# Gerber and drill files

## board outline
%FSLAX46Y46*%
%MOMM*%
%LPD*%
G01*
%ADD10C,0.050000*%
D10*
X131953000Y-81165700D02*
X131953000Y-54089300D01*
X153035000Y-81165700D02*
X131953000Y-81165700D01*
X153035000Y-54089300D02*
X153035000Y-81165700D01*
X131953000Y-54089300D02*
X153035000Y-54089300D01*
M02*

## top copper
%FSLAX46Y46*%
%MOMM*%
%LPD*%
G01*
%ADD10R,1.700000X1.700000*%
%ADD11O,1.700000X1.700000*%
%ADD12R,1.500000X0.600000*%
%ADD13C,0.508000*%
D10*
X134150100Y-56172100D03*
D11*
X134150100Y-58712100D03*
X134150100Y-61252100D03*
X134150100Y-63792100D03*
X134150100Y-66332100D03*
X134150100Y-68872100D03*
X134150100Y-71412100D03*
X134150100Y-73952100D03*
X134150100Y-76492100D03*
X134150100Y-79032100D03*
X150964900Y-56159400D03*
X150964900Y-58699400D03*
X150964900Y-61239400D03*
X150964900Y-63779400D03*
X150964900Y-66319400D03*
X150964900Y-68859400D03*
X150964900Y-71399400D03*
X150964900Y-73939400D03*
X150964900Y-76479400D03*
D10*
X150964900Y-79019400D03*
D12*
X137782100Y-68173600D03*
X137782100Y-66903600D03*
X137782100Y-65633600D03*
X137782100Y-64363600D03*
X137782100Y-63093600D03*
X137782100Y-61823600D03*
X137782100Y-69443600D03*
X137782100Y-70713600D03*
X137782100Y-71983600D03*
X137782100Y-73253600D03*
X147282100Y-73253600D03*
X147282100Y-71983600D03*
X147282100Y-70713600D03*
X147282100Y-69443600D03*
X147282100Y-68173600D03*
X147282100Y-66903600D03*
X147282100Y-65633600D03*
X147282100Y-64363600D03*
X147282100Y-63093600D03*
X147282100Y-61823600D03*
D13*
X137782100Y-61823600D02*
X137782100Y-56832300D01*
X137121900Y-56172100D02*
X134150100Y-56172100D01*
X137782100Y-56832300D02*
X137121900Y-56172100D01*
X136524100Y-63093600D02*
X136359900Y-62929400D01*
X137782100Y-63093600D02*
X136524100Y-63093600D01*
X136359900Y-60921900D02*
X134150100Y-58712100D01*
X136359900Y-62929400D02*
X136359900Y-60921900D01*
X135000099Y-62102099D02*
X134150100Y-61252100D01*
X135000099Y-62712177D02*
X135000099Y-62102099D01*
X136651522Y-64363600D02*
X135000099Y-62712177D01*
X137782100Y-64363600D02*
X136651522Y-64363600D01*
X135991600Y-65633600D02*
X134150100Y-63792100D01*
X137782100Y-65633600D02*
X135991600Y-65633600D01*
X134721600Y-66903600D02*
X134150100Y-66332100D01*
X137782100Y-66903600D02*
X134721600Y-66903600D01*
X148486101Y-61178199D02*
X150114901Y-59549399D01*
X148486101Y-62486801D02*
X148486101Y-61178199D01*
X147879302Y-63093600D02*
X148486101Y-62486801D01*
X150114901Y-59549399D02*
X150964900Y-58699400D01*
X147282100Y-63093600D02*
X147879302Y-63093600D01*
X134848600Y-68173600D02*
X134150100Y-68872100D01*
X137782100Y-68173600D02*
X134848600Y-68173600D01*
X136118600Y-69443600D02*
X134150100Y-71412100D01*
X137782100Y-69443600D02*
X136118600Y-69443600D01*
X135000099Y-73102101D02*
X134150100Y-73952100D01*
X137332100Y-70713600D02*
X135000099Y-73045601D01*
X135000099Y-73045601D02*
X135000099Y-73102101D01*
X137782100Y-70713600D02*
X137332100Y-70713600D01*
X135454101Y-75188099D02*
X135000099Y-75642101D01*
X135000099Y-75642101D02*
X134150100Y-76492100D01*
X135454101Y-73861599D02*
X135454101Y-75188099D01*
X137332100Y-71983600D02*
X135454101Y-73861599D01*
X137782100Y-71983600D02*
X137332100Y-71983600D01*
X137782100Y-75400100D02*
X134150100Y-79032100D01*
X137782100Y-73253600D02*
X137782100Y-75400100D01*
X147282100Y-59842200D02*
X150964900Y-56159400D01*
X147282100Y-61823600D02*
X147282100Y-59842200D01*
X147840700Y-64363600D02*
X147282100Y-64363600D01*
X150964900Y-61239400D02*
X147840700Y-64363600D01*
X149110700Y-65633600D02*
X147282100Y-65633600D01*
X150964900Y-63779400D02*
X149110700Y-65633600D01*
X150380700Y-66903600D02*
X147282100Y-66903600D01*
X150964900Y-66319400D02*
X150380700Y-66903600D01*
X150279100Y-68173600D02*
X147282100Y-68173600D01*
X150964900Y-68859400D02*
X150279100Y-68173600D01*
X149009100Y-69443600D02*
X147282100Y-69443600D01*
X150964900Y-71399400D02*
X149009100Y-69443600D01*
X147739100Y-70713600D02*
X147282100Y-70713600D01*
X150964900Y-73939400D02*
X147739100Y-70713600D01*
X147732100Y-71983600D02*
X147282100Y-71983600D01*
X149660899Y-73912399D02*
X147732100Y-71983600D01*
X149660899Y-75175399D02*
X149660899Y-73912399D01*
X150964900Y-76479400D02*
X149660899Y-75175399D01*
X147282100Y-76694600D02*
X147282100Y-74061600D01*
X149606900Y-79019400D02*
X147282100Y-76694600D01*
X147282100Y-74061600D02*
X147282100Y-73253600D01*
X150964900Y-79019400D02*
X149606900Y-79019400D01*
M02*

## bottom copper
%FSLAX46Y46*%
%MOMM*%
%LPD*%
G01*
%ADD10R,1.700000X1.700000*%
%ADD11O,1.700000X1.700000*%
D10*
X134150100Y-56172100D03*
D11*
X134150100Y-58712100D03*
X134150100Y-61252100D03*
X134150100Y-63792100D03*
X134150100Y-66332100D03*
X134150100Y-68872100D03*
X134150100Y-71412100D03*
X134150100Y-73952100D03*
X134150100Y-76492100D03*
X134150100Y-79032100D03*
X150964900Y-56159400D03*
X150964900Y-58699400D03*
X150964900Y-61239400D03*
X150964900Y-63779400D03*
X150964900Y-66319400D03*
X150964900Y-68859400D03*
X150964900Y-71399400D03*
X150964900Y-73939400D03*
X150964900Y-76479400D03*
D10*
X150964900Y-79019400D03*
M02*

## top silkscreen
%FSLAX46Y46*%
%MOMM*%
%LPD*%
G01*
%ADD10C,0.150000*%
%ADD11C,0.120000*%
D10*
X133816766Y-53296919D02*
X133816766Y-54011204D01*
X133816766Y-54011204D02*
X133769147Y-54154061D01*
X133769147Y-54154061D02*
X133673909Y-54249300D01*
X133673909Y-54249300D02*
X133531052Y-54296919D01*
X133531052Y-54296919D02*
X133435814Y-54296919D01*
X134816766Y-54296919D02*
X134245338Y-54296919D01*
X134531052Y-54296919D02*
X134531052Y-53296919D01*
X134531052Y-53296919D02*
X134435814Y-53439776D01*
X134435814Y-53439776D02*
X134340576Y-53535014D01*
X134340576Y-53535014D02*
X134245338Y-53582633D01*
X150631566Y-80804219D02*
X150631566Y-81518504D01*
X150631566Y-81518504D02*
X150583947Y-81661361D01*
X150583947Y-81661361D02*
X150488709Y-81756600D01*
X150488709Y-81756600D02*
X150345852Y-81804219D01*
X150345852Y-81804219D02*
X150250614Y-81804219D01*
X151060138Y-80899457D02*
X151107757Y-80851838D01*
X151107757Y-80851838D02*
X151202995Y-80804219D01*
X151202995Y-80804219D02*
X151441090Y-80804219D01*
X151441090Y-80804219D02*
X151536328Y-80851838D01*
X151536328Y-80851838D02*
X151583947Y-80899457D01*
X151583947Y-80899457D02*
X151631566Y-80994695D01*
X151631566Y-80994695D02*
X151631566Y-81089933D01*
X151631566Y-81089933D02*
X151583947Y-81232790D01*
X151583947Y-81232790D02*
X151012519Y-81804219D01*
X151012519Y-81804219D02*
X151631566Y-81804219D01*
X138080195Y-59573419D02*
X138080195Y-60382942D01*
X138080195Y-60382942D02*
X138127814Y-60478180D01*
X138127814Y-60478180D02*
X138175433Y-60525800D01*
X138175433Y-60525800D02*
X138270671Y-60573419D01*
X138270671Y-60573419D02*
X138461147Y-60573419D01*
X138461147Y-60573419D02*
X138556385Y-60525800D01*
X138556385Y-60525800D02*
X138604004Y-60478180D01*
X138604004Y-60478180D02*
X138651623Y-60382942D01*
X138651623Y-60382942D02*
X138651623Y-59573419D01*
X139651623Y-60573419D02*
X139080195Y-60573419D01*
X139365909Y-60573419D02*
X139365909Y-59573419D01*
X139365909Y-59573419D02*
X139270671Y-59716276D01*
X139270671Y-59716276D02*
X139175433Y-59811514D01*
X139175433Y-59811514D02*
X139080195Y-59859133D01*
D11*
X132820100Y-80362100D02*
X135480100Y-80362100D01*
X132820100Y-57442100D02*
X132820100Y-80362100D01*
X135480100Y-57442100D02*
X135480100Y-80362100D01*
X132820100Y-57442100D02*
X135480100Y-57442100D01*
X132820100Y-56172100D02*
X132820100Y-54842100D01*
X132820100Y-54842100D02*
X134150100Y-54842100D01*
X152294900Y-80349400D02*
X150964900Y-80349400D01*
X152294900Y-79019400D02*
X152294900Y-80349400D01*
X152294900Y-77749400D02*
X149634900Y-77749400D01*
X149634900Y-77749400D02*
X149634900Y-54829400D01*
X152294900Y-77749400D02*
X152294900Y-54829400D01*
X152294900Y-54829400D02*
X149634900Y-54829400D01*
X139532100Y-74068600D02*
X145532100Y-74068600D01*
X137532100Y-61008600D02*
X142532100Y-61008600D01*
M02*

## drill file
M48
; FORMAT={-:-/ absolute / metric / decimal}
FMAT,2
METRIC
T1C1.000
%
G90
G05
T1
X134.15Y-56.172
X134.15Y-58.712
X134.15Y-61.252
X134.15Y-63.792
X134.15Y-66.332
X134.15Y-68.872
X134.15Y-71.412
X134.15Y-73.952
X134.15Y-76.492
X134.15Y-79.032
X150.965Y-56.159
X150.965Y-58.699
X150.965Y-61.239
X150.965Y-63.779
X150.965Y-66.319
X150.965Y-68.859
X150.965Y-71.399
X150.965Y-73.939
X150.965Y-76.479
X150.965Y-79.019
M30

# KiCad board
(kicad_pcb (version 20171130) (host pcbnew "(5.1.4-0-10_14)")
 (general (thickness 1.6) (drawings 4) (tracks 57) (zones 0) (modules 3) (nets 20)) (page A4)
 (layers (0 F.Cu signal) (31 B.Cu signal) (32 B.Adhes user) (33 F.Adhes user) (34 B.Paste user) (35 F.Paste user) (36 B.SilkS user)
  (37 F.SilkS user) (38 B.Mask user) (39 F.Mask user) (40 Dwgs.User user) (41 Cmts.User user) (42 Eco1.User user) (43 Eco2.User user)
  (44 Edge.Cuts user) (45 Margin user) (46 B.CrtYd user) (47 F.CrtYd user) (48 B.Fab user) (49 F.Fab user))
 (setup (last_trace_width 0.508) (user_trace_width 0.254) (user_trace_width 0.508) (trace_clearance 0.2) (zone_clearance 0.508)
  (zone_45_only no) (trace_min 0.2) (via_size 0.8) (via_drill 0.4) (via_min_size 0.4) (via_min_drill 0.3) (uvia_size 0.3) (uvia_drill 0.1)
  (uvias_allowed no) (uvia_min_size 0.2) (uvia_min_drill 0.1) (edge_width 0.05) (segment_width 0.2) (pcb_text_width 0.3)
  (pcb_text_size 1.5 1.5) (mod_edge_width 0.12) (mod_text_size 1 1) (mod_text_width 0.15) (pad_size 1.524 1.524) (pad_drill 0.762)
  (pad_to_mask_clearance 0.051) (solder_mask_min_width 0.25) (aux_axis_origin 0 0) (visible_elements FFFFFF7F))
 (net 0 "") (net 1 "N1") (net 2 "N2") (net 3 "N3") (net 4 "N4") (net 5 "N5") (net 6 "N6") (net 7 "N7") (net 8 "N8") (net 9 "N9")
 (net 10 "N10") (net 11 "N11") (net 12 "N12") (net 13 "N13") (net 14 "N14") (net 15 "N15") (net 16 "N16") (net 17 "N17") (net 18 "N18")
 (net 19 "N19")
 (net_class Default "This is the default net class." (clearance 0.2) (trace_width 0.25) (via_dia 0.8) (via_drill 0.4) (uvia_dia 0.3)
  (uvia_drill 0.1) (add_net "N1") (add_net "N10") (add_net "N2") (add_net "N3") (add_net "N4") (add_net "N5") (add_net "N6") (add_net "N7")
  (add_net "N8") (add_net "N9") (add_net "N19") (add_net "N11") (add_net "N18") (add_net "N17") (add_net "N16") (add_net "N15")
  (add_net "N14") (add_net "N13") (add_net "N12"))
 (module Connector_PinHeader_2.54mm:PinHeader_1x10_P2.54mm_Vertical (layer F.Cu) (at 134.1501 56.1721)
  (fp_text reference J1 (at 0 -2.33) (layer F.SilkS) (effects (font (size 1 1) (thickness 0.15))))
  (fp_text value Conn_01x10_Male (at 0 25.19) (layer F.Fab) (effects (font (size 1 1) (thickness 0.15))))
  (fp_line (start -1.33 24.19) (end 1.33 24.19) (layer F.SilkS) (width 0.12))
  (fp_line (start -1.33 1.27) (end -1.33 24.19) (layer F.SilkS) (width 0.12))
  (fp_line (start 1.33 1.27) (end 1.33 24.19) (layer F.SilkS) (width 0.12))
  (fp_line (start -1.33 1.27) (end 1.33 1.27) (layer F.SilkS) (width 0.12))
  (fp_line (start -1.33 0) (end -1.33 -1.33) (layer F.SilkS) (width 0.12))
  (fp_line (start -1.33 -1.33) (end 0 -1.33) (layer F.SilkS) (width 0.12))
  (pad 1 thru_hole rect (at 0 0) (size 1.7 1.7) (drill 1) (layers *.Cu *.Mask) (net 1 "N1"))
  (pad 2 thru_hole oval (at 0 2.54) (size 1.7 1.7) (drill 1) (layers *.Cu *.Mask) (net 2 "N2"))
  (pad 3 thru_hole oval (at 0 5.08) (size 1.7 1.7) (drill 1) (layers *.Cu *.Mask) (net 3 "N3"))
  (pad 4 thru_hole oval (at 0 7.62) (size 1.7 1.7) (drill 1) (layers *.Cu *.Mask) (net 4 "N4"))
  (pad 5 thru_hole oval (at 0 10.16) (size 1.7 1.7) (drill 1) (layers *.Cu *.Mask) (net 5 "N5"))
  (pad 6 thru_hole oval (at 0 12.7) (size 1.7 1.7) (drill 1) (layers *.Cu *.Mask) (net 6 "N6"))
  (pad 7 thru_hole oval (at 0 15.24) (size 1.7 1.7) (drill 1) (layers *.Cu *.Mask) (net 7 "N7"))
  (pad 8 thru_hole oval (at 0 17.78) (size 1.7 1.7) (drill 1) (layers *.Cu *.Mask) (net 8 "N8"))
  (pad 9 thru_hole oval (at 0 20.32) (size 1.7 1.7) (drill 1) (layers *.Cu *.Mask) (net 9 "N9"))
  (pad 10 thru_hole oval (at 0 22.86) (size 1.7 1.7) (drill 1) (layers *.Cu *.Mask) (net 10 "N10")))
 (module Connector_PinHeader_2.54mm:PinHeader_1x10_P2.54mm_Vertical (layer F.Cu) (at 150.9649 79.0194 180)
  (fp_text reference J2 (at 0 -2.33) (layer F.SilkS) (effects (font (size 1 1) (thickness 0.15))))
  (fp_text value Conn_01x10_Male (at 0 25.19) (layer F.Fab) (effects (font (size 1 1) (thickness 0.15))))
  (fp_line (start -1.33 -1.33) (end 0 -1.33) (layer F.SilkS) (width 0.12))
  (fp_line (start -1.33 0) (end -1.33 -1.33) (layer F.SilkS) (width 0.12))
  (fp_line (start -1.33 1.27) (end 1.33 1.27) (layer F.SilkS) (width 0.12))
  (fp_line (start 1.33 1.27) (end 1.33 24.19) (layer F.SilkS) (width 0.12))
  (fp_line (start -1.33 1.27) (end -1.33 24.19) (layer F.SilkS) (width 0.12))
  (fp_line (start -1.33 24.19) (end 1.33 24.19) (layer F.SilkS) (width 0.12))
  (pad 10 thru_hole oval (at 0 22.86 180) (size 1.7 1.7) (drill 1) (layers *.Cu *.Mask) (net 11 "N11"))
  (pad 9 thru_hole oval (at 0 20.32 180) (size 1.7 1.7) (drill 1) (layers *.Cu *.Mask) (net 5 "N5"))
  (pad 8 thru_hole oval (at 0 17.78 180) (size 1.7 1.7) (drill 1) (layers *.Cu *.Mask) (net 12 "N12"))
  (pad 7 thru_hole oval (at 0 15.24 180) (size 1.7 1.7) (drill 1) (layers *.Cu *.Mask) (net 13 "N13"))
  (pad 6 thru_hole oval (at 0 12.7 180) (size 1.7 1.7) (drill 1) (layers *.Cu *.Mask) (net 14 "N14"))
  (pad 5 thru_hole oval (at 0 10.16 180) (size 1.7 1.7) (drill 1) (layers *.Cu *.Mask) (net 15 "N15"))
  (pad 4 thru_hole oval (at 0 7.62 180) (size 1.7 1.7) (drill 1) (layers *.Cu *.Mask) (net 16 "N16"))
  (pad 3 thru_hole oval (at 0 5.08 180) (size 1.7 1.7) (drill 1) (layers *.Cu *.Mask) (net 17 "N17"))
  (pad 2 thru_hole oval (at 0 2.54 180) (size 1.7 1.7) (drill 1) (layers *.Cu *.Mask) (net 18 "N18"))
  (pad 1 thru_hole rect (at 0 0 180) (size 1.7 1.7) (drill 1) (layers *.Cu *.Mask) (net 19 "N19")))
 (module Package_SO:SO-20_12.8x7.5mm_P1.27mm (layer F.Cu) (at 142.5321 67.5386)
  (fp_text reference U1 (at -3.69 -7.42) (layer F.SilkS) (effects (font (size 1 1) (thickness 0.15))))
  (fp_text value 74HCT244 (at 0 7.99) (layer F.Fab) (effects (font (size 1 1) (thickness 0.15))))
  (fp_line (start -3 6.53) (end 3 6.53) (layer F.SilkS) (width 0.12))
  (fp_line (start -5 -6.53) (end 0 -6.53) (layer F.SilkS) (width 0.12))
  (pad 6 smd rect (at -4.75 0.635) (size 1.5 0.6) (layers F.Cu F.Paste F.Mask) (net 6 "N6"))
  (pad 5 smd rect (at -4.75 -0.635) (size 1.5 0.6) (layers F.Cu F.Paste F.Mask) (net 5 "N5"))
  (pad 4 smd rect (at -4.75 -1.905) (size 1.5 0.6) (layers F.Cu F.Paste F.Mask) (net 4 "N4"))
  (pad 3 smd rect (at -4.75 -3.175) (size 1.5 0.6) (layers F.Cu F.Paste F.Mask) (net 3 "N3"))
  (pad 2 smd rect (at -4.75 -4.445) (size 1.5 0.6) (layers F.Cu F.Paste F.Mask) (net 2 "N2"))
  (pad 1 smd rect (at -4.75 -5.715) (size 1.5 0.6) (layers F.Cu F.Paste F.Mask) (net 1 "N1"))
  (pad 7 smd rect (at -4.75 1.905) (size 1.5 0.6) (layers F.Cu F.Paste F.Mask) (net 7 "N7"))
  (pad 8 smd rect (at -4.75 3.175) (size 1.5 0.6) (layers F.Cu F.Paste F.Mask) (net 8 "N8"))
  (pad 9 smd rect (at -4.75 4.445) (size 1.5 0.6) (layers F.Cu F.Paste F.Mask) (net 9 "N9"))
  (pad 10 smd rect (at -4.75 5.715) (size 1.5 0.6) (layers F.Cu F.Paste F.Mask) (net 10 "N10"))
  (pad 11 smd rect (at 4.75 5.715) (size 1.5 0.6) (layers F.Cu F.Paste F.Mask) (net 19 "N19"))
  (pad 12 smd rect (at 4.75 4.445) (size 1.5 0.6) (layers F.Cu F.Paste F.Mask) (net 18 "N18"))
  (pad 13 smd rect (at 4.75 3.175) (size 1.5 0.6) (layers F.Cu F.Paste F.Mask) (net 17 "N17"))
  (pad 14 smd rect (at 4.75 1.905) (size 1.5 0.6) (layers F.Cu F.Paste F.Mask) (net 16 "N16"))
  (pad 15 smd rect (at 4.75 0.635) (size 1.5 0.6) (layers F.Cu F.Paste F.Mask) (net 15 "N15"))
  (pad 16 smd rect (at 4.75 -0.635) (size 1.5 0.6) (layers F.Cu F.Paste F.Mask) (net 14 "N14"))
  (pad 17 smd rect (at 4.75 -1.905) (size 1.5 0.6) (layers F.Cu F.Paste F.Mask) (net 13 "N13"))
  (pad 18 smd rect (at 4.75 -3.175) (size 1.5 0.6) (layers F.Cu F.Paste F.Mask) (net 12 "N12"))
  (pad 19 smd rect (at 4.75 -4.445) (size 1.5 0.6) (layers F.Cu F.Paste F.Mask) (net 5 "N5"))
  (pad 20 smd rect (at 4.75 -5.715) (size 1.5 0.6) (layers F.Cu F.Paste F.Mask) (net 11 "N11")))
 (gr_line (start 131.953 81.1657) (end 131.953 54.0893) (layer Edge.Cuts) (width 0.05))
 (gr_line (start 153.035 81.1657) (end 131.953 81.1657) (layer Edge.Cuts) (width 0.05))
 (gr_line (start 153.035 54.0893) (end 153.035 81.1657) (layer Edge.Cuts) (width 0.05))
 (gr_line (start 131.953 54.0893) (end 153.035 54.0893) (layer Edge.Cuts) (width 0.05))
 (segment (start 137.7821 61.8236) (end 137.7821 56.8323) (width 0.508) (layer F.Cu) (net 1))
 (segment (start 137.1219 56.1721) (end 134.1501 56.1721) (width 0.508) (layer F.Cu) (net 1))
 (segment (start 137.7821 56.8323) (end 137.1219 56.1721) (width 0.508) (layer F.Cu) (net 1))
 (segment (start 136.5241 63.0936) (end 136.3599 62.9294) (width 0.508) (layer F.Cu) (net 2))
 (segment (start 137.7821 63.0936) (end 136.5241 63.0936) (width 0.508) (layer F.Cu) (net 2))
 (segment (start 136.3599 60.9219) (end 134.1501 58.7121) (width 0.508) (layer F.Cu) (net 2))
 (segment (start 136.3599 62.9294) (end 136.3599 60.9219) (width 0.508) (layer F.Cu) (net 2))
 (segment (start 135.000099 62.102099) (end 134.1501 61.2521) (width 0.508) (layer F.Cu) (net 3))
 (segment (start 135.000099 62.712177) (end 135.000099 62.102099) (width 0.508) (layer F.Cu) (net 3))
 (segment (start 136.651522 64.3636) (end 135.000099 62.712177) (width 0.508) (layer F.Cu) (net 3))
 (segment (start 137.7821 64.3636) (end 136.651522 64.3636) (width 0.508) (layer F.Cu) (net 3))
 (segment (start 135.9916 65.6336) (end 134.1501 63.7921) (width 0.508) (layer F.Cu) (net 4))
 (segment (start 137.7821 65.6336) (end 135.9916 65.6336) (width 0.508) (layer F.Cu) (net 4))
 (segment (start 134.7216 66.9036) (end 134.1501 66.3321) (width 0.508) (layer F.Cu) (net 5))
 (segment (start 137.7821 66.9036) (end 134.7216 66.9036) (width 0.508) (layer F.Cu) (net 5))
 (segment (start 148.486101 61.178199) (end 150.114901 59.549399) (width 0.508) (layer F.Cu) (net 5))
 (segment (start 148.486101 62.486801) (end 148.486101 61.178199) (width 0.508) (layer F.Cu) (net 5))
 (segment (start 147.879302 63.0936) (end 148.486101 62.486801) (width 0.508) (layer F.Cu) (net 5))
 (segment (start 150.114901 59.549399) (end 150.9649 58.6994) (width 0.508) (layer F.Cu) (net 5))
 (segment (start 147.2821 63.0936) (end 147.879302 63.0936) (width 0.508) (layer F.Cu) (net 5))
 (segment (start 134.8486 68.1736) (end 134.1501 68.8721) (width 0.508) (layer F.Cu) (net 6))
 (segment (start 137.7821 68.1736) (end 134.8486 68.1736) (width 0.508) (layer F.Cu) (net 6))
 (segment (start 136.1186 69.4436) (end 134.1501 71.4121) (width 0.508) (layer F.Cu) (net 7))
 (segment (start 137.7821 69.4436) (end 136.1186 69.4436) (width 0.508) (layer F.Cu) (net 7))
 (segment (start 135.000099 73.102101) (end 134.1501 73.9521) (width 0.508) (layer F.Cu) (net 8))
 (segment (start 137.3321 70.7136) (end 135.000099 73.045601) (width 0.508) (layer F.Cu) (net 8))
 (segment (start 135.000099 73.045601) (end 135.000099 73.102101) (width 0.508) (layer F.Cu) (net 8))
 (segment (start 137.7821 70.7136) (end 137.3321 70.7136) (width 0.508) (layer F.Cu) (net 8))
 (segment (start 135.454101 75.188099) (end 135.000099 75.642101) (width 0.508) (layer F.Cu) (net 9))
 (segment (start 135.000099 75.642101) (end 134.1501 76.4921) (width 0.508) (layer F.Cu) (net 9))
 (segment (start 135.454101 73.861599) (end 135.454101 75.188099) (width 0.508) (layer F.Cu) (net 9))
 (segment (start 137.3321 71.9836) (end 135.454101 73.861599) (width 0.508) (layer F.Cu) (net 9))
 (segment (start 137.7821 71.9836) (end 137.3321 71.9836) (width 0.508) (layer F.Cu) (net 9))
 (segment (start 137.7821 75.4001) (end 134.1501 79.0321) (width 0.508) (layer F.Cu) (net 10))
 (segment (start 137.7821 73.2536) (end 137.7821 75.4001) (width 0.508) (layer F.Cu) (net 10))
 (segment (start 147.2821 59.8422) (end 150.9649 56.1594) (width 0.508) (layer F.Cu) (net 11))
 (segment (start 147.2821 61.8236) (end 147.2821 59.8422) (width 0.508) (layer F.Cu) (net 11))
 (segment (start 147.8407 64.3636) (end 147.2821 64.3636) (width 0.508) (layer F.Cu) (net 12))
 (segment (start 150.9649 61.2394) (end 147.8407 64.3636) (width 0.508) (layer F.Cu) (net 12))
 (segment (start 149.1107 65.6336) (end 147.2821 65.6336) (width 0.508) (layer F.Cu) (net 13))
 (segment (start 150.9649 63.7794) (end 149.1107 65.6336) (width 0.508) (layer F.Cu) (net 13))
 (segment (start 150.3807 66.9036) (end 147.2821 66.9036) (width 0.508) (layer F.Cu) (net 14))
 (segment (start 150.9649 66.3194) (end 150.3807 66.9036) (width 0.508) (layer F.Cu) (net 14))
 (segment (start 150.2791 68.1736) (end 147.2821 68.1736) (width 0.508) (layer F.Cu) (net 15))
 (segment (start 150.9649 68.8594) (end 150.2791 68.1736) (width 0.508) (layer F.Cu) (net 15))
 (segment (start 149.0091 69.4436) (end 147.2821 69.4436) (width 0.508) (layer F.Cu) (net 16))
 (segment (start 150.9649 71.3994) (end 149.0091 69.4436) (width 0.508) (layer F.Cu) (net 16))
 (segment (start 147.7391 70.7136) (end 147.2821 70.7136) (width 0.508) (layer F.Cu) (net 17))
 (segment (start 150.9649 73.9394) (end 147.7391 70.7136) (width 0.508) (layer F.Cu) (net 17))
 (segment (start 147.7321 71.9836) (end 147.2821 71.9836) (width 0.508) (layer F.Cu) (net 18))
 (segment (start 149.660899 73.912399) (end 147.7321 71.9836) (width 0.508) (layer F.Cu) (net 18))
 (segment (start 149.660899 75.175399) (end 149.660899 73.912399) (width 0.508) (layer F.Cu) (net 18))
 (segment (start 150.9649 76.4794) (end 149.660899 75.175399) (width 0.508) (layer F.Cu) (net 18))
 (segment (start 147.2821 76.6946) (end 147.2821 74.0616) (width 0.508) (layer F.Cu) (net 19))
 (segment (start 149.6069 79.0194) (end 147.2821 76.6946) (width 0.508) (layer F.Cu) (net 19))
 (segment (start 147.2821 74.0616) (end 147.2821 73.2536) (width 0.508) (layer F.Cu) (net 19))
 (segment (start 150.9649 79.0194) (end 149.6069 79.0194) (width 0.508) (layer F.Cu) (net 19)))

